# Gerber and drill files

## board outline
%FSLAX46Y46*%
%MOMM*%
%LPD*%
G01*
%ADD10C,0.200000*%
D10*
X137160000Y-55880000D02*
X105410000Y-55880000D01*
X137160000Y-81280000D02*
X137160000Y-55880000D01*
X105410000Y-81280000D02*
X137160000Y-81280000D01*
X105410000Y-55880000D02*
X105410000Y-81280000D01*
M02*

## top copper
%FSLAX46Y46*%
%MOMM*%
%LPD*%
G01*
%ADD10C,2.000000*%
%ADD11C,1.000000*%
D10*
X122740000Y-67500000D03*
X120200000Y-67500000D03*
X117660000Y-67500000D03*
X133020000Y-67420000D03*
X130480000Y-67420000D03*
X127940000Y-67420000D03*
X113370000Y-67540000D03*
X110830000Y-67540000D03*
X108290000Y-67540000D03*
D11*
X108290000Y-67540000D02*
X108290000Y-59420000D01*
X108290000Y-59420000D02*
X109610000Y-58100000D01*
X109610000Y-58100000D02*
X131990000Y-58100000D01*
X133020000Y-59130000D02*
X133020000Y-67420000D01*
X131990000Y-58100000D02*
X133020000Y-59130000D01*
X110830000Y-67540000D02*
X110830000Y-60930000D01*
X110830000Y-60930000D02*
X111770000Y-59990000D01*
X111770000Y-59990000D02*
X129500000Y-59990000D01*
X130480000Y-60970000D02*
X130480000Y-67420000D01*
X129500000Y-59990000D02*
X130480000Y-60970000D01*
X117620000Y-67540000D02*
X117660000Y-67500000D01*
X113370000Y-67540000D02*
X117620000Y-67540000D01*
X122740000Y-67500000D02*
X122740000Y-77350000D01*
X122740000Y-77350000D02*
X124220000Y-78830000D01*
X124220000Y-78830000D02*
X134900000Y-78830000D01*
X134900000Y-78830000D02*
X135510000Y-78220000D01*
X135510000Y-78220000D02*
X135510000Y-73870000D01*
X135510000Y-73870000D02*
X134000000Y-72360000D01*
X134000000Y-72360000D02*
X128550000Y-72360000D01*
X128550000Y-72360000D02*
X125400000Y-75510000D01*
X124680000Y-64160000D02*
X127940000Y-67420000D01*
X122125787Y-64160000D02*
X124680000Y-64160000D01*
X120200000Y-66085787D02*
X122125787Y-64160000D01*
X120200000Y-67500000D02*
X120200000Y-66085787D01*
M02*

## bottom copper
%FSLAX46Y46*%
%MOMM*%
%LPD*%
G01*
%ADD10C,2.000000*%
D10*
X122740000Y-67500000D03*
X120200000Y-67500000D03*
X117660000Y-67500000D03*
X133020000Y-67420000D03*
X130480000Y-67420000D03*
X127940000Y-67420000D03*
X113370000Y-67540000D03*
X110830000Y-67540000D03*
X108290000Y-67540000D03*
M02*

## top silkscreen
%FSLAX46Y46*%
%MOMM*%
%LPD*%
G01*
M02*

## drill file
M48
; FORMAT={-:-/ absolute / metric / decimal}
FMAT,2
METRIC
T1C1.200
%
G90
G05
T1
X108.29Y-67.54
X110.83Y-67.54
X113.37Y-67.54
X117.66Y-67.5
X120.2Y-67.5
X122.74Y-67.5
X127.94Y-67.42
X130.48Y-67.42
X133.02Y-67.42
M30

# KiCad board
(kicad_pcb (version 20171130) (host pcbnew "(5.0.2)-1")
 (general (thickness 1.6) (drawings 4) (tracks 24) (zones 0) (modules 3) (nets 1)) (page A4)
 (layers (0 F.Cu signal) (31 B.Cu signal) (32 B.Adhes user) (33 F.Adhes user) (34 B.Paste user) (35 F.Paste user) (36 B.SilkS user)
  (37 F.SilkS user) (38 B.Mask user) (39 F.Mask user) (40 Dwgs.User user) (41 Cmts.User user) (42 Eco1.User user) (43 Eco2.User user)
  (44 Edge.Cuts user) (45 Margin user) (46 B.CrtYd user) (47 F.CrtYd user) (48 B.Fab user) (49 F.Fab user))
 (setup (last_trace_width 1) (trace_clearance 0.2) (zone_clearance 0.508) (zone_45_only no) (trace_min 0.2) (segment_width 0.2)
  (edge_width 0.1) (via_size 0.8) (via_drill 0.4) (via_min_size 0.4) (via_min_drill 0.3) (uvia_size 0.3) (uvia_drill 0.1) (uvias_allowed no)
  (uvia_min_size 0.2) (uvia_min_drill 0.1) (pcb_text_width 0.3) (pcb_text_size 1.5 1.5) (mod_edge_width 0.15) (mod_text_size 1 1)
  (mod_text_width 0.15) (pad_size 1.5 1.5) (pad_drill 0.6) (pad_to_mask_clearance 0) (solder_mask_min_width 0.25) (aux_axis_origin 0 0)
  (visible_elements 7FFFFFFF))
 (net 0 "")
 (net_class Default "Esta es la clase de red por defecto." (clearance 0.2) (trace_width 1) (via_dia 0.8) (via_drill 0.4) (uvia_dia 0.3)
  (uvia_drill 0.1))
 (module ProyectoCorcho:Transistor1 (layer F.Cu) (at 120.2 67.5)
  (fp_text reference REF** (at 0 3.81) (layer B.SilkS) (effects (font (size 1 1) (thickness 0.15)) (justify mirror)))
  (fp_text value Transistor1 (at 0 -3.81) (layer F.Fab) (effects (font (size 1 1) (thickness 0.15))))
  (pad 3 thru_hole circle (at 2.54 0) (size 2 2) (drill 1.2) (layers *.Cu *.Mask))
  (pad 2 thru_hole circle (at 0 0) (size 2 2) (drill 1.2) (layers *.Cu *.Mask))
  (pad 1 thru_hole circle (at -2.54 0) (size 2 2) (drill 1.2) (layers *.Cu *.Mask)))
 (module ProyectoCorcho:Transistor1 (layer F.Cu) (at 130.48 67.42)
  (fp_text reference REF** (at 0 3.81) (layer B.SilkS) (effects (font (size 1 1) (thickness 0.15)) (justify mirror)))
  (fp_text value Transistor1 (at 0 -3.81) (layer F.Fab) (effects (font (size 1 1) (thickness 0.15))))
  (pad 3 thru_hole circle (at 2.54 0) (size 2 2) (drill 1.2) (layers *.Cu *.Mask))
  (pad 2 thru_hole circle (at 0 0) (size 2 2) (drill 1.2) (layers *.Cu *.Mask))
  (pad 1 thru_hole circle (at -2.54 0) (size 2 2) (drill 1.2) (layers *.Cu *.Mask)))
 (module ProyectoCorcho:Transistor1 (layer F.Cu) (at 110.83 67.54)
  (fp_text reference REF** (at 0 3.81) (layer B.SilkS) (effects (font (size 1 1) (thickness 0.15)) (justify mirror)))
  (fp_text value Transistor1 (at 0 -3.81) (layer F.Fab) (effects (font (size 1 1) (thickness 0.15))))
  (pad 3 thru_hole circle (at 2.54 0) (size 2 2) (drill 1.2) (layers *.Cu *.Mask))
  (pad 2 thru_hole circle (at 0 0) (size 2 2) (drill 1.2) (layers *.Cu *.Mask))
  (pad 1 thru_hole circle (at -2.54 0) (size 2 2) (drill 1.2) (layers *.Cu *.Mask)))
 (gr_line (start 137.16 55.88) (end 105.41 55.88) (layer Edge.Cuts) (width 0.2))
 (gr_line (start 137.16 81.28) (end 137.16 55.88) (layer Edge.Cuts) (width 0.2))
 (gr_line (start 105.41 81.28) (end 137.16 81.28) (layer Edge.Cuts) (width 0.2))
 (gr_line (start 105.41 55.88) (end 105.41 81.28) (layer Edge.Cuts) (width 0.2))
 (segment (start 108.29 67.54) (end 108.29 59.42) (width 1) (layer F.Cu) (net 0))
 (segment (start 108.29 59.42) (end 109.61 58.1) (width 1) (layer F.Cu) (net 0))
 (segment (start 109.61 58.1) (end 131.99 58.1) (width 1) (layer F.Cu) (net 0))
 (segment (start 133.02 59.13) (end 133.02 67.42) (width 1) (layer F.Cu) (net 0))
 (segment (start 131.99 58.1) (end 133.02 59.13) (width 1) (layer F.Cu) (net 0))
 (segment (start 110.83 67.54) (end 110.83 60.93) (width 1) (layer F.Cu) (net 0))
 (segment (start 110.83 60.93) (end 111.77 59.99) (width 1) (layer F.Cu) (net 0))
 (segment (start 111.77 59.99) (end 129.5 59.99) (width 1) (layer F.Cu) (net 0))
 (segment (start 130.48 60.97) (end 130.48 67.42) (width 1) (layer F.Cu) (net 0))
 (segment (start 129.5 59.99) (end 130.48 60.97) (width 1) (layer F.Cu) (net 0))
 (segment (start 117.62 67.54) (end 117.66 67.5) (width 1) (layer F.Cu) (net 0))
 (segment (start 113.37 67.54) (end 117.62 67.54) (width 1) (layer F.Cu) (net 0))
 (segment (start 122.74 67.5) (end 122.74 77.35) (width 1) (layer F.Cu) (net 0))
 (segment (start 122.74 77.35) (end 124.22 78.83) (width 1) (layer F.Cu) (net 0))
 (segment (start 124.22 78.83) (end 134.9 78.83) (width 1) (layer F.Cu) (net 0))
 (segment (start 134.9 78.83) (end 135.51 78.22) (width 1) (layer F.Cu) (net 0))
 (segment (start 135.51 78.22) (end 135.51 73.87) (width 1) (layer F.Cu) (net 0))
 (segment (start 135.51 73.87) (end 134 72.36) (width 1) (layer F.Cu) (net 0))
 (segment (start 134 72.36) (end 128.55 72.36) (width 1) (layer F.Cu) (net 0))
 (segment (start 128.55 72.36) (end 125.4 75.51) (width 1) (layer F.Cu) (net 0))
 (segment (start 124.68 64.16) (end 127.94 67.42) (width 1) (layer F.Cu) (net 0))
 (segment (start 122.125787 64.16) (end 124.68 64.16) (width 1) (layer F.Cu) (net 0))
 (segment (start 120.2 66.085787) (end 122.125787 64.16) (width 1) (layer F.Cu) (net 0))
 (segment (start 120.2 67.5) (end 120.2 66.085787) (width 1) (layer F.Cu) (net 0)))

